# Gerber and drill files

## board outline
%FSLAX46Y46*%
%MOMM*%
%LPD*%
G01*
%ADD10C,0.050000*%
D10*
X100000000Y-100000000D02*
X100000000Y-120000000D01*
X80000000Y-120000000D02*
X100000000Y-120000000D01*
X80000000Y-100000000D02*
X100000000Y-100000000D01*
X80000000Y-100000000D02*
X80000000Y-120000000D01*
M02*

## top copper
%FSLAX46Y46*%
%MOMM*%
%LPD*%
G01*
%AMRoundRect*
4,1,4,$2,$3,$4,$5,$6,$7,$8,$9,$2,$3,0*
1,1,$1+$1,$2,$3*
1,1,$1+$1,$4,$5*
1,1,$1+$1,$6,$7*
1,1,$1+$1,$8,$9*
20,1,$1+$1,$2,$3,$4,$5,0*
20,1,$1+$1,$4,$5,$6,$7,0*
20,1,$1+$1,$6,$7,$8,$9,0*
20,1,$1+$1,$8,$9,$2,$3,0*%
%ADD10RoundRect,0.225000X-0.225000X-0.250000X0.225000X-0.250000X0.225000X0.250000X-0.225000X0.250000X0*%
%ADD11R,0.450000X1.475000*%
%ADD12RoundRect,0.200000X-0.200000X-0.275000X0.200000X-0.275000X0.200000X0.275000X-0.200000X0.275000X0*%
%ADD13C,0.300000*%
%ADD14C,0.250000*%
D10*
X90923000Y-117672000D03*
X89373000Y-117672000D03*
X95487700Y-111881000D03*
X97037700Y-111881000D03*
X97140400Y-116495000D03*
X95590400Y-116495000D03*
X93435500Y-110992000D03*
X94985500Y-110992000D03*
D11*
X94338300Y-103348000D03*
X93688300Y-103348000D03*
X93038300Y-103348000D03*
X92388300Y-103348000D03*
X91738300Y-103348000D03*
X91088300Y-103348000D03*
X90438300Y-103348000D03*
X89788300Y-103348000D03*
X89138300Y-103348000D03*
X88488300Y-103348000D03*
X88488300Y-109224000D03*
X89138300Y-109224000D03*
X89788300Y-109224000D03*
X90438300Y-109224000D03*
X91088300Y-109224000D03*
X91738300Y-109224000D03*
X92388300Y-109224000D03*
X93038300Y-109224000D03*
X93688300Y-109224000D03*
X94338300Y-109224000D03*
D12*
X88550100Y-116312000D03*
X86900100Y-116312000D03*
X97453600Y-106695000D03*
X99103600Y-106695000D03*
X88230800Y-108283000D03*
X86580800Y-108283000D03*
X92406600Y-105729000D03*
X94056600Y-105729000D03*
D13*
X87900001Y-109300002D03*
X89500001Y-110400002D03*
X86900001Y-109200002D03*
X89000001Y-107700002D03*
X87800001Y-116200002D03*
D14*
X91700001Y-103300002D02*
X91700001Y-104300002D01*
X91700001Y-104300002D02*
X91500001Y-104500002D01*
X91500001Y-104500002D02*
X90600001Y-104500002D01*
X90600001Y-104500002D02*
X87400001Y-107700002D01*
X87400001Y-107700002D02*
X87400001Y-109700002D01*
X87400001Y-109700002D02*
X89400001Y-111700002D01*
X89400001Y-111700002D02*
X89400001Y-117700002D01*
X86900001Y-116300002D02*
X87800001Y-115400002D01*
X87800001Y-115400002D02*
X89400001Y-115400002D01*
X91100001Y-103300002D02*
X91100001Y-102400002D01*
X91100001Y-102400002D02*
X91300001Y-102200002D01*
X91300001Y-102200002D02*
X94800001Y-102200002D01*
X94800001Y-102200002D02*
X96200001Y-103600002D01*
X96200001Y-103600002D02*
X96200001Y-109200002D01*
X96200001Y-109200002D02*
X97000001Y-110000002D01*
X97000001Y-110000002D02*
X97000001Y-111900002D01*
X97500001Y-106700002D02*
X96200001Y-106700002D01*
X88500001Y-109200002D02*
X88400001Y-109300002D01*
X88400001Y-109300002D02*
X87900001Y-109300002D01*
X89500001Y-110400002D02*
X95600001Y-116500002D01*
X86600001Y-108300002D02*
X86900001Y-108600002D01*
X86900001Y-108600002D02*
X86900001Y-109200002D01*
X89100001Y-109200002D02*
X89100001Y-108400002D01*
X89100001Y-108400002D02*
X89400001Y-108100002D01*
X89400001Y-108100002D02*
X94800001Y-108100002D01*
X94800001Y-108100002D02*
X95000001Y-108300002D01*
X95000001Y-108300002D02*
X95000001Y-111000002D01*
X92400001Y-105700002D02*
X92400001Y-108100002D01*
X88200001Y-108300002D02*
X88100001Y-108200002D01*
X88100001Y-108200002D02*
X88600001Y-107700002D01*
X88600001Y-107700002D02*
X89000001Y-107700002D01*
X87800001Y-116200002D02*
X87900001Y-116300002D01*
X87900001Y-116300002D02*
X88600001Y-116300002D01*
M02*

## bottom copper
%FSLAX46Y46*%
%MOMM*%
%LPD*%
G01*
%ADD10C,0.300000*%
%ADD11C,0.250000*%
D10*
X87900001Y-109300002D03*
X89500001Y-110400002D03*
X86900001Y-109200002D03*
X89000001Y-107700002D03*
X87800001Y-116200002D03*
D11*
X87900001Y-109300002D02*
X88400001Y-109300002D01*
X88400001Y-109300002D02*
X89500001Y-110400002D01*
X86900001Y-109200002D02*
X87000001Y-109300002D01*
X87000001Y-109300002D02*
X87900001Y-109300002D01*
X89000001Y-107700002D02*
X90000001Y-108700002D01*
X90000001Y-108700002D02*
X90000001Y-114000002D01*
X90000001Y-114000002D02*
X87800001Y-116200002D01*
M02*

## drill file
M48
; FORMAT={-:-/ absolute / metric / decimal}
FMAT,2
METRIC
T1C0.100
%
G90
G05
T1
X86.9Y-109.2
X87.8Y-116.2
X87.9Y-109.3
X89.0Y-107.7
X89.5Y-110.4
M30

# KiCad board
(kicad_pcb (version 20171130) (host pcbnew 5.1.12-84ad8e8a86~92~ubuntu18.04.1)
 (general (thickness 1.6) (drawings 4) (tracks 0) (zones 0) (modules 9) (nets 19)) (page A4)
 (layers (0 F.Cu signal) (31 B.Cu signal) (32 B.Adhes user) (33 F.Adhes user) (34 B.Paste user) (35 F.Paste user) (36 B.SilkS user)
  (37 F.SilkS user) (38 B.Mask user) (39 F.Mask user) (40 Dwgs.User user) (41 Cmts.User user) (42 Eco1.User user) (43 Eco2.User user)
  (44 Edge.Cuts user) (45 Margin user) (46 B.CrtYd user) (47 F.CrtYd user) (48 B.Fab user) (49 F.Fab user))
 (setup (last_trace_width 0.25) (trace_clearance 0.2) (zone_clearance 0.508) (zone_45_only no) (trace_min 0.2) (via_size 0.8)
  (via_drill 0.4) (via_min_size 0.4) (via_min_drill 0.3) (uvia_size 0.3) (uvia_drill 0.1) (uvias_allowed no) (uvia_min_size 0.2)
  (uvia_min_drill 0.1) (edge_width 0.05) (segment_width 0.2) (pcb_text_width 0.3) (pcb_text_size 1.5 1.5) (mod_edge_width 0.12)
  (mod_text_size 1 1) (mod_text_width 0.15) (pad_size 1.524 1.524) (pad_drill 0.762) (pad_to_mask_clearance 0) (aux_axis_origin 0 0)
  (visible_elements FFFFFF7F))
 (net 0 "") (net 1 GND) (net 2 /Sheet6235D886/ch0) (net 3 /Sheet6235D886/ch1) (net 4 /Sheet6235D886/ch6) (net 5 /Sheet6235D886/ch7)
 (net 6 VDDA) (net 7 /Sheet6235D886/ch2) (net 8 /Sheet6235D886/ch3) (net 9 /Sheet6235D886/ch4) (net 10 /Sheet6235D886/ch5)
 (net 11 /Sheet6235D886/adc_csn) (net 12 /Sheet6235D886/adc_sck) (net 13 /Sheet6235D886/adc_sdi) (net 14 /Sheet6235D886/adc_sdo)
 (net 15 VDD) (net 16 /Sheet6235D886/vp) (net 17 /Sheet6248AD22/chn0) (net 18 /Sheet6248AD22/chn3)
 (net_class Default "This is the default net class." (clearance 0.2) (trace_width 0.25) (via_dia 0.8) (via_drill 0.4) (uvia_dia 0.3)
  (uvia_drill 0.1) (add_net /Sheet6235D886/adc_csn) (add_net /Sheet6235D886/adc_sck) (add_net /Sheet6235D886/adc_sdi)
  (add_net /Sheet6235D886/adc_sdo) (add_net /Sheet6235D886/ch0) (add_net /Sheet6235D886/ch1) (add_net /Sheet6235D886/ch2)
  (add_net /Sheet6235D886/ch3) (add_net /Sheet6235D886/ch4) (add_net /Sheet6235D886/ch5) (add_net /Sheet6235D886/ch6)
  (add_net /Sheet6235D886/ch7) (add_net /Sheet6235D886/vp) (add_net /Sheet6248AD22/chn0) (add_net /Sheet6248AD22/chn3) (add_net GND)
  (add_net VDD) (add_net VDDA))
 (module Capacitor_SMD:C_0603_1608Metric (layer F.Cu) (at 90.148000 117.672000)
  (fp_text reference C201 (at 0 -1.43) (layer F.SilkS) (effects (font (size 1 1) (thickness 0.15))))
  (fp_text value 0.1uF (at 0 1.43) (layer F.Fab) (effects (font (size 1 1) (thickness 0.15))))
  (pad 2 smd roundrect (at 0.775 0) (size 0.9 0.95) (layers F.Cu F.Mask F.Paste) (roundrect_rratio 0.25) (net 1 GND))
  (pad 1 smd roundrect (at -0.775 0) (size 0.9 0.95) (layers F.Cu F.Mask F.Paste) (roundrect_rratio 0.25) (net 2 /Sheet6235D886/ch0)))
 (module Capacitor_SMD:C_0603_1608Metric (layer F.Cu) (at 96.262700 111.881000)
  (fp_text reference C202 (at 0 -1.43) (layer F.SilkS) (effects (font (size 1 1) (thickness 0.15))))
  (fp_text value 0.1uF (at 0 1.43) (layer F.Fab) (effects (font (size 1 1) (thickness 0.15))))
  (pad 1 smd roundrect (at -0.775 0) (size 0.9 0.95) (layers F.Cu F.Mask F.Paste) (roundrect_rratio 0.25) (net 1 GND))
  (pad 2 smd roundrect (at 0.775 0) (size 0.9 0.95) (layers F.Cu F.Mask F.Paste) (roundrect_rratio 0.25) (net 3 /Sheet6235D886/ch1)))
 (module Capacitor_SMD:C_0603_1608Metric (layer F.Cu) (at 96.365400 116.495000)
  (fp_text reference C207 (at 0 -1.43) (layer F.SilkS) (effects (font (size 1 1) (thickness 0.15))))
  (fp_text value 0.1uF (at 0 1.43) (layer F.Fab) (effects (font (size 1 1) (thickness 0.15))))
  (pad 2 smd roundrect (at 0.775 0) (size 0.9 0.95) (layers F.Cu F.Mask F.Paste) (roundrect_rratio 0.25) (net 1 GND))
  (pad 1 smd roundrect (at -0.775 0) (size 0.9 0.95) (layers F.Cu F.Mask F.Paste) (roundrect_rratio 0.25) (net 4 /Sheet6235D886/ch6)))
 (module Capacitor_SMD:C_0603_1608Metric (layer F.Cu) (at 94.210500 110.992000)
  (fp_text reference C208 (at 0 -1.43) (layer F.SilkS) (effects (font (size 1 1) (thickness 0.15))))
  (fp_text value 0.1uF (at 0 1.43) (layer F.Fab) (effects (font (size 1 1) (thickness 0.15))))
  (pad 1 smd roundrect (at -0.775 0) (size 0.9 0.95) (layers F.Cu F.Mask F.Paste) (roundrect_rratio 0.25) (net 1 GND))
  (pad 2 smd roundrect (at 0.775 0) (size 0.9 0.95) (layers F.Cu F.Mask F.Paste) (roundrect_rratio 0.25) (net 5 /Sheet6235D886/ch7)))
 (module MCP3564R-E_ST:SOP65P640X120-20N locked (layer F.Cu) (at 91.413300 106.286000 270.000000)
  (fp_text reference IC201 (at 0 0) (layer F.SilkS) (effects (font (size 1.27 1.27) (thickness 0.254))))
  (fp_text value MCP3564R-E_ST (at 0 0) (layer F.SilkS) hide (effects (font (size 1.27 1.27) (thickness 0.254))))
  (pad 1 smd rect (at -2.938 -2.925) (size 0.45 1.475) (layers F.Cu F.Mask F.Paste) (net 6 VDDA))
  (pad 2 smd rect (at -2.938 -2.275) (size 0.45 1.475) (layers F.Cu F.Mask F.Paste) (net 1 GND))
  (pad 3 smd rect (at -2.938 -1.625) (size 0.45 1.475) (layers F.Cu F.Mask F.Paste) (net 1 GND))
  (pad 4 smd rect (at -2.938 -0.975) (size 0.45 1.475) (layers F.Cu F.Mask F.Paste))
  (pad 5 smd rect (at -2.938 -0.325) (size 0.45 1.475) (layers F.Cu F.Mask F.Paste) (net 2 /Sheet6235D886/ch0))
  (pad 6 smd rect (at -2.938 0.325) (size 0.45 1.475) (layers F.Cu F.Mask F.Paste) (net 3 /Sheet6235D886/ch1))
  (pad 7 smd rect (at -2.938 0.975) (size 0.45 1.475) (layers F.Cu F.Mask F.Paste) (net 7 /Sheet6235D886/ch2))
  (pad 8 smd rect (at -2.938 1.625) (size 0.45 1.475) (layers F.Cu F.Mask F.Paste) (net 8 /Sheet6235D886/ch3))
  (pad 9 smd rect (at -2.938 2.275) (size 0.45 1.475) (layers F.Cu F.Mask F.Paste) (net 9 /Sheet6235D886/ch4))
  (pad 10 smd rect (at -2.938 2.925) (size 0.45 1.475) (layers F.Cu F.Mask F.Paste) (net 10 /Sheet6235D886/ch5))
  (pad 11 smd rect (at 2.938 2.925) (size 0.45 1.475) (layers F.Cu F.Mask F.Paste) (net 4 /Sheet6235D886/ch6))
  (pad 12 smd rect (at 2.938 2.275) (size 0.45 1.475) (layers F.Cu F.Mask F.Paste) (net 5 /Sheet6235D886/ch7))
  (pad 13 smd rect (at 2.938 1.625) (size 0.45 1.475) (layers F.Cu F.Mask F.Paste) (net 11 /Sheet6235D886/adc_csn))
  (pad 14 smd rect (at 2.938 0.975) (size 0.45 1.475) (layers F.Cu F.Mask F.Paste) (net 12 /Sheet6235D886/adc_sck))
  (pad 15 smd rect (at 2.938 0.325) (size 0.45 1.475) (layers F.Cu F.Mask F.Paste) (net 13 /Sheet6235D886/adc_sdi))
  (pad 16 smd rect (at 2.938 -0.325) (size 0.45 1.475) (layers F.Cu F.Mask F.Paste) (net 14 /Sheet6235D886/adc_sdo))
  (pad 17 smd rect (at 2.938 -0.975) (size 0.45 1.475) (layers F.Cu F.Mask F.Paste))
  (pad 18 smd rect (at 2.938 -1.625) (size 0.45 1.475) (layers F.Cu F.Mask F.Paste))
  (pad 19 smd rect (at 2.938 -2.275) (size 0.45 1.475) (layers F.Cu F.Mask F.Paste) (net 1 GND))
  (pad 20 smd rect (at 2.938 -2.925) (size 0.45 1.475) (layers F.Cu F.Mask F.Paste) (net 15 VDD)))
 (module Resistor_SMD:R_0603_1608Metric (layer F.Cu) (at 87.725100 116.312000)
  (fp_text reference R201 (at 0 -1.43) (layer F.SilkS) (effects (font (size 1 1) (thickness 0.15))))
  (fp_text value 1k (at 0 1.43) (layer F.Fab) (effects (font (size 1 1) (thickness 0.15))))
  (pad 2 smd roundrect (at 0.825 0) (size 0.8 0.95) (layers F.Cu F.Mask F.Paste) (roundrect_rratio 0.25) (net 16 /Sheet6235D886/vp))
  (pad 1 smd roundrect (at -0.825 0) (size 0.8 0.95) (layers F.Cu F.Mask F.Paste) (roundrect_rratio 0.25) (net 2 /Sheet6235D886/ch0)))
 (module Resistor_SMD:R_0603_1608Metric (layer F.Cu) (at 98.278600 106.695000)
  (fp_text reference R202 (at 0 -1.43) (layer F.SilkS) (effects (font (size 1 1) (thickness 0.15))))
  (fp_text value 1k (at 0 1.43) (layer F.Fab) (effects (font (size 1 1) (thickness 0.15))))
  (pad 1 smd roundrect (at -0.825 0) (size 0.8 0.95) (layers F.Cu F.Mask F.Paste) (roundrect_rratio 0.25) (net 3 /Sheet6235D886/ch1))
  (pad 2 smd roundrect (at 0.825 0) (size 0.8 0.95) (layers F.Cu F.Mask F.Paste) (roundrect_rratio 0.25) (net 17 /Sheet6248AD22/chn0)))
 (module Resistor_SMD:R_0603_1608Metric (layer F.Cu) (at 87.405800 108.283000)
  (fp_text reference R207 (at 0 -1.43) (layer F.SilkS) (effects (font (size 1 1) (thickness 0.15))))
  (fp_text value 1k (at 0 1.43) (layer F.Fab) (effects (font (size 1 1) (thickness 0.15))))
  (pad 2 smd roundrect (at 0.825 0) (size 0.8 0.95) (layers F.Cu F.Mask F.Paste) (roundrect_rratio 0.25) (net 16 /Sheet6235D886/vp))
  (pad 1 smd roundrect (at -0.825 0) (size 0.8 0.95) (layers F.Cu F.Mask F.Paste) (roundrect_rratio 0.25) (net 4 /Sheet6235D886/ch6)))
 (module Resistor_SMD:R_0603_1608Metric (layer F.Cu) (at 93.231600 105.729000)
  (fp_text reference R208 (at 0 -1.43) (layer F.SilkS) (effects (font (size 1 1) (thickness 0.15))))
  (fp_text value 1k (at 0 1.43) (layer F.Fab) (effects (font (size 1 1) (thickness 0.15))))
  (pad 1 smd roundrect (at -0.825 0) (size 0.8 0.95) (layers F.Cu F.Mask F.Paste) (roundrect_rratio 0.25) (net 5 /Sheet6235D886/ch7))
  (pad 2 smd roundrect (at 0.825 0) (size 0.8 0.95) (layers F.Cu F.Mask F.Paste) (roundrect_rratio 0.25) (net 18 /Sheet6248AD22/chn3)))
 (gr_line (start 100 100) (end 100 120) (layer Edge.Cuts) (width 0.05))
 (gr_line (start 80 120) (end 100 120) (layer Edge.Cuts) (width 0.05))
 (gr_line (start 80 100) (end 100 100) (layer Edge.Cuts) (width 0.05))
 (gr_line (start 80 100) (end 80 120) (layer Edge.Cuts) (width 0.05))
 (segment (start 91.700001 103.300002) (end 91.700001 104.300002) (width 0.250000) (layer F.Cu) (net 2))
 (segment (start 91.700001 104.300002) (end 91.500001 104.500002) (width 0.250000) (layer F.Cu) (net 2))
 (segment (start 91.500001 104.500002) (end 90.600001 104.500002) (width 0.250000) (layer F.Cu) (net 2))
 (segment (start 90.600001 104.500002) (end 87.400001 107.700002) (width 0.250000) (layer F.Cu) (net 2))
 (segment (start 87.400001 107.700002) (end 87.400001 109.700002) (width 0.250000) (layer F.Cu) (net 2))
 (segment (start 87.400001 109.700002) (end 89.400001 111.700002) (width 0.250000) (layer F.Cu) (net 2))
 (segment (start 89.400001 111.700002) (end 89.400001 117.700002) (width 0.250000) (layer F.Cu) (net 2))
 (segment (start 86.900001 116.300002) (end 87.800001 115.400002) (width 0.250000) (layer F.Cu) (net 2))
 (segment (start 87.800001 115.400002) (end 89.400001 115.400002) (width 0.250000) (layer F.Cu) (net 2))
 (segment (start 91.100001 103.300002) (end 91.100001 102.400002) (width 0.250000) (layer F.Cu) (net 3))
 (segment (start 91.100001 102.400002) (end 91.300001 102.200002) (width 0.250000) (layer F.Cu) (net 3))
 (segment (start 91.300001 102.200002) (end 94.800001 102.200002) (width 0.250000) (layer F.Cu) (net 3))
 (segment (start 94.800001 102.200002) (end 96.200001 103.600002) (width 0.250000) (layer F.Cu) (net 3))
 (segment (start 96.200001 103.600002) (end 96.200001 109.200002) (width 0.250000) (layer F.Cu) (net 3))
 (segment (start 96.200001 109.200002) (end 97.000001 110.000002) (width 0.250000) (layer F.Cu) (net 3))
 (segment (start 97.000001 110.000002) (end 97.000001 111.900002) (width 0.250000) (layer F.Cu) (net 3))
 (segment (start 97.500001 106.700002) (end 96.200001 106.700002) (width 0.250000) (layer F.Cu) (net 3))
 (segment (start 88.500001 109.200002) (end 88.400001 109.300002) (width 0.250000) (layer F.Cu) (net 4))
 (segment (start 88.400001 109.300002) (end 87.900001 109.300002) (width 0.250000) (layer F.Cu) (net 4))
 (segment (start 87.900001 109.300002) (end 88.400001 109.300002) (width 0.250000) (layer B.Cu) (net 4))
 (segment (start 88.400001 109.300002) (end 89.500001 110.400002) (width 0.250000) (layer B.Cu) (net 4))
 (segment (start 89.500001 110.400002) (end 95.600001 116.500002) (width 0.250000) (layer F.Cu) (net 4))
 (segment (start 86.600001 108.300002) (end 86.900001 108.600002) (width 0.250000) (layer F.Cu) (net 4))
 (segment (start 86.900001 108.600002) (end 86.900001 109.200002) (width 0.250000) (layer F.Cu) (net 4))
 (segment (start 86.900001 109.200002) (end 87.000001 109.300002) (width 0.250000) (layer B.Cu) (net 4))
 (segment (start 87.000001 109.300002) (end 87.900001 109.300002) (width 0.250000) (layer B.Cu) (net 4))
 (via micro (at 87.900001 109.300002) (size 0.300000) (drill 0.100000) (layers F.Cu B.Cu) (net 4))
 (via micro (at 89.500001 110.400002) (size 0.300000) (drill 0.100000) (layers F.Cu B.Cu) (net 4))
 (via micro (at 86.900001 109.200002) (size 0.300000) (drill 0.100000) (layers F.Cu B.Cu) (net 4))
 (segment (start 89.100001 109.200002) (end 89.100001 108.400002) (width 0.250000) (layer F.Cu) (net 5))
 (segment (start 89.100001 108.400002) (end 89.400001 108.100002) (width 0.250000) (layer F.Cu) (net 5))
 (segment (start 89.400001 108.100002) (end 94.800001 108.100002) (width 0.250000) (layer F.Cu) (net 5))
 (segment (start 94.800001 108.100002) (end 95.000001 108.300002) (width 0.250000) (layer F.Cu) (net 5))
 (segment (start 95.000001 108.300002) (end 95.000001 111.000002) (width 0.250000) (layer F.Cu) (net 5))
 (segment (start 92.400001 105.700002) (end 92.400001 108.100002) (width 0.250000) (layer F.Cu) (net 5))
 (segment (start 88.200001 108.300002) (end 88.100001 108.200002) (width 0.250000) (layer F.Cu) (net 16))
 (segment (start 88.100001 108.200002) (end 88.600001 107.700002) (width 0.250000) (layer F.Cu) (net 16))
 (segment (start 88.600001 107.700002) (end 89.000001 107.700002) (width 0.250000) (layer F.Cu) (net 16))
 (segment (start 89.000001 107.700002) (end 90.000001 108.700002) (width 0.250000) (layer B.Cu) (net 16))
 (segment (start 90.000001 108.700002) (end 90.000001 114.000002) (width 0.250000) (layer B.Cu) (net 16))
 (segment (start 90.000001 114.000002) (end 87.800001 116.200002) (width 0.250000) (layer B.Cu) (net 16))
 (segment (start 87.800001 116.200002) (end 87.900001 116.300002) (width 0.250000) (layer F.Cu) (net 16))
 (segment (start 87.900001 116.300002) (end 88.600001 116.300002) (width 0.250000) (layer F.Cu) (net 16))
 (via micro (at 89.000001 107.700002) (size 0.300000) (drill 0.100000) (layers F.Cu B.Cu) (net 16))
 (via micro (at 87.800001 116.200002) (size 0.300000) (drill 0.100000) (layers F.Cu B.Cu) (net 16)))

